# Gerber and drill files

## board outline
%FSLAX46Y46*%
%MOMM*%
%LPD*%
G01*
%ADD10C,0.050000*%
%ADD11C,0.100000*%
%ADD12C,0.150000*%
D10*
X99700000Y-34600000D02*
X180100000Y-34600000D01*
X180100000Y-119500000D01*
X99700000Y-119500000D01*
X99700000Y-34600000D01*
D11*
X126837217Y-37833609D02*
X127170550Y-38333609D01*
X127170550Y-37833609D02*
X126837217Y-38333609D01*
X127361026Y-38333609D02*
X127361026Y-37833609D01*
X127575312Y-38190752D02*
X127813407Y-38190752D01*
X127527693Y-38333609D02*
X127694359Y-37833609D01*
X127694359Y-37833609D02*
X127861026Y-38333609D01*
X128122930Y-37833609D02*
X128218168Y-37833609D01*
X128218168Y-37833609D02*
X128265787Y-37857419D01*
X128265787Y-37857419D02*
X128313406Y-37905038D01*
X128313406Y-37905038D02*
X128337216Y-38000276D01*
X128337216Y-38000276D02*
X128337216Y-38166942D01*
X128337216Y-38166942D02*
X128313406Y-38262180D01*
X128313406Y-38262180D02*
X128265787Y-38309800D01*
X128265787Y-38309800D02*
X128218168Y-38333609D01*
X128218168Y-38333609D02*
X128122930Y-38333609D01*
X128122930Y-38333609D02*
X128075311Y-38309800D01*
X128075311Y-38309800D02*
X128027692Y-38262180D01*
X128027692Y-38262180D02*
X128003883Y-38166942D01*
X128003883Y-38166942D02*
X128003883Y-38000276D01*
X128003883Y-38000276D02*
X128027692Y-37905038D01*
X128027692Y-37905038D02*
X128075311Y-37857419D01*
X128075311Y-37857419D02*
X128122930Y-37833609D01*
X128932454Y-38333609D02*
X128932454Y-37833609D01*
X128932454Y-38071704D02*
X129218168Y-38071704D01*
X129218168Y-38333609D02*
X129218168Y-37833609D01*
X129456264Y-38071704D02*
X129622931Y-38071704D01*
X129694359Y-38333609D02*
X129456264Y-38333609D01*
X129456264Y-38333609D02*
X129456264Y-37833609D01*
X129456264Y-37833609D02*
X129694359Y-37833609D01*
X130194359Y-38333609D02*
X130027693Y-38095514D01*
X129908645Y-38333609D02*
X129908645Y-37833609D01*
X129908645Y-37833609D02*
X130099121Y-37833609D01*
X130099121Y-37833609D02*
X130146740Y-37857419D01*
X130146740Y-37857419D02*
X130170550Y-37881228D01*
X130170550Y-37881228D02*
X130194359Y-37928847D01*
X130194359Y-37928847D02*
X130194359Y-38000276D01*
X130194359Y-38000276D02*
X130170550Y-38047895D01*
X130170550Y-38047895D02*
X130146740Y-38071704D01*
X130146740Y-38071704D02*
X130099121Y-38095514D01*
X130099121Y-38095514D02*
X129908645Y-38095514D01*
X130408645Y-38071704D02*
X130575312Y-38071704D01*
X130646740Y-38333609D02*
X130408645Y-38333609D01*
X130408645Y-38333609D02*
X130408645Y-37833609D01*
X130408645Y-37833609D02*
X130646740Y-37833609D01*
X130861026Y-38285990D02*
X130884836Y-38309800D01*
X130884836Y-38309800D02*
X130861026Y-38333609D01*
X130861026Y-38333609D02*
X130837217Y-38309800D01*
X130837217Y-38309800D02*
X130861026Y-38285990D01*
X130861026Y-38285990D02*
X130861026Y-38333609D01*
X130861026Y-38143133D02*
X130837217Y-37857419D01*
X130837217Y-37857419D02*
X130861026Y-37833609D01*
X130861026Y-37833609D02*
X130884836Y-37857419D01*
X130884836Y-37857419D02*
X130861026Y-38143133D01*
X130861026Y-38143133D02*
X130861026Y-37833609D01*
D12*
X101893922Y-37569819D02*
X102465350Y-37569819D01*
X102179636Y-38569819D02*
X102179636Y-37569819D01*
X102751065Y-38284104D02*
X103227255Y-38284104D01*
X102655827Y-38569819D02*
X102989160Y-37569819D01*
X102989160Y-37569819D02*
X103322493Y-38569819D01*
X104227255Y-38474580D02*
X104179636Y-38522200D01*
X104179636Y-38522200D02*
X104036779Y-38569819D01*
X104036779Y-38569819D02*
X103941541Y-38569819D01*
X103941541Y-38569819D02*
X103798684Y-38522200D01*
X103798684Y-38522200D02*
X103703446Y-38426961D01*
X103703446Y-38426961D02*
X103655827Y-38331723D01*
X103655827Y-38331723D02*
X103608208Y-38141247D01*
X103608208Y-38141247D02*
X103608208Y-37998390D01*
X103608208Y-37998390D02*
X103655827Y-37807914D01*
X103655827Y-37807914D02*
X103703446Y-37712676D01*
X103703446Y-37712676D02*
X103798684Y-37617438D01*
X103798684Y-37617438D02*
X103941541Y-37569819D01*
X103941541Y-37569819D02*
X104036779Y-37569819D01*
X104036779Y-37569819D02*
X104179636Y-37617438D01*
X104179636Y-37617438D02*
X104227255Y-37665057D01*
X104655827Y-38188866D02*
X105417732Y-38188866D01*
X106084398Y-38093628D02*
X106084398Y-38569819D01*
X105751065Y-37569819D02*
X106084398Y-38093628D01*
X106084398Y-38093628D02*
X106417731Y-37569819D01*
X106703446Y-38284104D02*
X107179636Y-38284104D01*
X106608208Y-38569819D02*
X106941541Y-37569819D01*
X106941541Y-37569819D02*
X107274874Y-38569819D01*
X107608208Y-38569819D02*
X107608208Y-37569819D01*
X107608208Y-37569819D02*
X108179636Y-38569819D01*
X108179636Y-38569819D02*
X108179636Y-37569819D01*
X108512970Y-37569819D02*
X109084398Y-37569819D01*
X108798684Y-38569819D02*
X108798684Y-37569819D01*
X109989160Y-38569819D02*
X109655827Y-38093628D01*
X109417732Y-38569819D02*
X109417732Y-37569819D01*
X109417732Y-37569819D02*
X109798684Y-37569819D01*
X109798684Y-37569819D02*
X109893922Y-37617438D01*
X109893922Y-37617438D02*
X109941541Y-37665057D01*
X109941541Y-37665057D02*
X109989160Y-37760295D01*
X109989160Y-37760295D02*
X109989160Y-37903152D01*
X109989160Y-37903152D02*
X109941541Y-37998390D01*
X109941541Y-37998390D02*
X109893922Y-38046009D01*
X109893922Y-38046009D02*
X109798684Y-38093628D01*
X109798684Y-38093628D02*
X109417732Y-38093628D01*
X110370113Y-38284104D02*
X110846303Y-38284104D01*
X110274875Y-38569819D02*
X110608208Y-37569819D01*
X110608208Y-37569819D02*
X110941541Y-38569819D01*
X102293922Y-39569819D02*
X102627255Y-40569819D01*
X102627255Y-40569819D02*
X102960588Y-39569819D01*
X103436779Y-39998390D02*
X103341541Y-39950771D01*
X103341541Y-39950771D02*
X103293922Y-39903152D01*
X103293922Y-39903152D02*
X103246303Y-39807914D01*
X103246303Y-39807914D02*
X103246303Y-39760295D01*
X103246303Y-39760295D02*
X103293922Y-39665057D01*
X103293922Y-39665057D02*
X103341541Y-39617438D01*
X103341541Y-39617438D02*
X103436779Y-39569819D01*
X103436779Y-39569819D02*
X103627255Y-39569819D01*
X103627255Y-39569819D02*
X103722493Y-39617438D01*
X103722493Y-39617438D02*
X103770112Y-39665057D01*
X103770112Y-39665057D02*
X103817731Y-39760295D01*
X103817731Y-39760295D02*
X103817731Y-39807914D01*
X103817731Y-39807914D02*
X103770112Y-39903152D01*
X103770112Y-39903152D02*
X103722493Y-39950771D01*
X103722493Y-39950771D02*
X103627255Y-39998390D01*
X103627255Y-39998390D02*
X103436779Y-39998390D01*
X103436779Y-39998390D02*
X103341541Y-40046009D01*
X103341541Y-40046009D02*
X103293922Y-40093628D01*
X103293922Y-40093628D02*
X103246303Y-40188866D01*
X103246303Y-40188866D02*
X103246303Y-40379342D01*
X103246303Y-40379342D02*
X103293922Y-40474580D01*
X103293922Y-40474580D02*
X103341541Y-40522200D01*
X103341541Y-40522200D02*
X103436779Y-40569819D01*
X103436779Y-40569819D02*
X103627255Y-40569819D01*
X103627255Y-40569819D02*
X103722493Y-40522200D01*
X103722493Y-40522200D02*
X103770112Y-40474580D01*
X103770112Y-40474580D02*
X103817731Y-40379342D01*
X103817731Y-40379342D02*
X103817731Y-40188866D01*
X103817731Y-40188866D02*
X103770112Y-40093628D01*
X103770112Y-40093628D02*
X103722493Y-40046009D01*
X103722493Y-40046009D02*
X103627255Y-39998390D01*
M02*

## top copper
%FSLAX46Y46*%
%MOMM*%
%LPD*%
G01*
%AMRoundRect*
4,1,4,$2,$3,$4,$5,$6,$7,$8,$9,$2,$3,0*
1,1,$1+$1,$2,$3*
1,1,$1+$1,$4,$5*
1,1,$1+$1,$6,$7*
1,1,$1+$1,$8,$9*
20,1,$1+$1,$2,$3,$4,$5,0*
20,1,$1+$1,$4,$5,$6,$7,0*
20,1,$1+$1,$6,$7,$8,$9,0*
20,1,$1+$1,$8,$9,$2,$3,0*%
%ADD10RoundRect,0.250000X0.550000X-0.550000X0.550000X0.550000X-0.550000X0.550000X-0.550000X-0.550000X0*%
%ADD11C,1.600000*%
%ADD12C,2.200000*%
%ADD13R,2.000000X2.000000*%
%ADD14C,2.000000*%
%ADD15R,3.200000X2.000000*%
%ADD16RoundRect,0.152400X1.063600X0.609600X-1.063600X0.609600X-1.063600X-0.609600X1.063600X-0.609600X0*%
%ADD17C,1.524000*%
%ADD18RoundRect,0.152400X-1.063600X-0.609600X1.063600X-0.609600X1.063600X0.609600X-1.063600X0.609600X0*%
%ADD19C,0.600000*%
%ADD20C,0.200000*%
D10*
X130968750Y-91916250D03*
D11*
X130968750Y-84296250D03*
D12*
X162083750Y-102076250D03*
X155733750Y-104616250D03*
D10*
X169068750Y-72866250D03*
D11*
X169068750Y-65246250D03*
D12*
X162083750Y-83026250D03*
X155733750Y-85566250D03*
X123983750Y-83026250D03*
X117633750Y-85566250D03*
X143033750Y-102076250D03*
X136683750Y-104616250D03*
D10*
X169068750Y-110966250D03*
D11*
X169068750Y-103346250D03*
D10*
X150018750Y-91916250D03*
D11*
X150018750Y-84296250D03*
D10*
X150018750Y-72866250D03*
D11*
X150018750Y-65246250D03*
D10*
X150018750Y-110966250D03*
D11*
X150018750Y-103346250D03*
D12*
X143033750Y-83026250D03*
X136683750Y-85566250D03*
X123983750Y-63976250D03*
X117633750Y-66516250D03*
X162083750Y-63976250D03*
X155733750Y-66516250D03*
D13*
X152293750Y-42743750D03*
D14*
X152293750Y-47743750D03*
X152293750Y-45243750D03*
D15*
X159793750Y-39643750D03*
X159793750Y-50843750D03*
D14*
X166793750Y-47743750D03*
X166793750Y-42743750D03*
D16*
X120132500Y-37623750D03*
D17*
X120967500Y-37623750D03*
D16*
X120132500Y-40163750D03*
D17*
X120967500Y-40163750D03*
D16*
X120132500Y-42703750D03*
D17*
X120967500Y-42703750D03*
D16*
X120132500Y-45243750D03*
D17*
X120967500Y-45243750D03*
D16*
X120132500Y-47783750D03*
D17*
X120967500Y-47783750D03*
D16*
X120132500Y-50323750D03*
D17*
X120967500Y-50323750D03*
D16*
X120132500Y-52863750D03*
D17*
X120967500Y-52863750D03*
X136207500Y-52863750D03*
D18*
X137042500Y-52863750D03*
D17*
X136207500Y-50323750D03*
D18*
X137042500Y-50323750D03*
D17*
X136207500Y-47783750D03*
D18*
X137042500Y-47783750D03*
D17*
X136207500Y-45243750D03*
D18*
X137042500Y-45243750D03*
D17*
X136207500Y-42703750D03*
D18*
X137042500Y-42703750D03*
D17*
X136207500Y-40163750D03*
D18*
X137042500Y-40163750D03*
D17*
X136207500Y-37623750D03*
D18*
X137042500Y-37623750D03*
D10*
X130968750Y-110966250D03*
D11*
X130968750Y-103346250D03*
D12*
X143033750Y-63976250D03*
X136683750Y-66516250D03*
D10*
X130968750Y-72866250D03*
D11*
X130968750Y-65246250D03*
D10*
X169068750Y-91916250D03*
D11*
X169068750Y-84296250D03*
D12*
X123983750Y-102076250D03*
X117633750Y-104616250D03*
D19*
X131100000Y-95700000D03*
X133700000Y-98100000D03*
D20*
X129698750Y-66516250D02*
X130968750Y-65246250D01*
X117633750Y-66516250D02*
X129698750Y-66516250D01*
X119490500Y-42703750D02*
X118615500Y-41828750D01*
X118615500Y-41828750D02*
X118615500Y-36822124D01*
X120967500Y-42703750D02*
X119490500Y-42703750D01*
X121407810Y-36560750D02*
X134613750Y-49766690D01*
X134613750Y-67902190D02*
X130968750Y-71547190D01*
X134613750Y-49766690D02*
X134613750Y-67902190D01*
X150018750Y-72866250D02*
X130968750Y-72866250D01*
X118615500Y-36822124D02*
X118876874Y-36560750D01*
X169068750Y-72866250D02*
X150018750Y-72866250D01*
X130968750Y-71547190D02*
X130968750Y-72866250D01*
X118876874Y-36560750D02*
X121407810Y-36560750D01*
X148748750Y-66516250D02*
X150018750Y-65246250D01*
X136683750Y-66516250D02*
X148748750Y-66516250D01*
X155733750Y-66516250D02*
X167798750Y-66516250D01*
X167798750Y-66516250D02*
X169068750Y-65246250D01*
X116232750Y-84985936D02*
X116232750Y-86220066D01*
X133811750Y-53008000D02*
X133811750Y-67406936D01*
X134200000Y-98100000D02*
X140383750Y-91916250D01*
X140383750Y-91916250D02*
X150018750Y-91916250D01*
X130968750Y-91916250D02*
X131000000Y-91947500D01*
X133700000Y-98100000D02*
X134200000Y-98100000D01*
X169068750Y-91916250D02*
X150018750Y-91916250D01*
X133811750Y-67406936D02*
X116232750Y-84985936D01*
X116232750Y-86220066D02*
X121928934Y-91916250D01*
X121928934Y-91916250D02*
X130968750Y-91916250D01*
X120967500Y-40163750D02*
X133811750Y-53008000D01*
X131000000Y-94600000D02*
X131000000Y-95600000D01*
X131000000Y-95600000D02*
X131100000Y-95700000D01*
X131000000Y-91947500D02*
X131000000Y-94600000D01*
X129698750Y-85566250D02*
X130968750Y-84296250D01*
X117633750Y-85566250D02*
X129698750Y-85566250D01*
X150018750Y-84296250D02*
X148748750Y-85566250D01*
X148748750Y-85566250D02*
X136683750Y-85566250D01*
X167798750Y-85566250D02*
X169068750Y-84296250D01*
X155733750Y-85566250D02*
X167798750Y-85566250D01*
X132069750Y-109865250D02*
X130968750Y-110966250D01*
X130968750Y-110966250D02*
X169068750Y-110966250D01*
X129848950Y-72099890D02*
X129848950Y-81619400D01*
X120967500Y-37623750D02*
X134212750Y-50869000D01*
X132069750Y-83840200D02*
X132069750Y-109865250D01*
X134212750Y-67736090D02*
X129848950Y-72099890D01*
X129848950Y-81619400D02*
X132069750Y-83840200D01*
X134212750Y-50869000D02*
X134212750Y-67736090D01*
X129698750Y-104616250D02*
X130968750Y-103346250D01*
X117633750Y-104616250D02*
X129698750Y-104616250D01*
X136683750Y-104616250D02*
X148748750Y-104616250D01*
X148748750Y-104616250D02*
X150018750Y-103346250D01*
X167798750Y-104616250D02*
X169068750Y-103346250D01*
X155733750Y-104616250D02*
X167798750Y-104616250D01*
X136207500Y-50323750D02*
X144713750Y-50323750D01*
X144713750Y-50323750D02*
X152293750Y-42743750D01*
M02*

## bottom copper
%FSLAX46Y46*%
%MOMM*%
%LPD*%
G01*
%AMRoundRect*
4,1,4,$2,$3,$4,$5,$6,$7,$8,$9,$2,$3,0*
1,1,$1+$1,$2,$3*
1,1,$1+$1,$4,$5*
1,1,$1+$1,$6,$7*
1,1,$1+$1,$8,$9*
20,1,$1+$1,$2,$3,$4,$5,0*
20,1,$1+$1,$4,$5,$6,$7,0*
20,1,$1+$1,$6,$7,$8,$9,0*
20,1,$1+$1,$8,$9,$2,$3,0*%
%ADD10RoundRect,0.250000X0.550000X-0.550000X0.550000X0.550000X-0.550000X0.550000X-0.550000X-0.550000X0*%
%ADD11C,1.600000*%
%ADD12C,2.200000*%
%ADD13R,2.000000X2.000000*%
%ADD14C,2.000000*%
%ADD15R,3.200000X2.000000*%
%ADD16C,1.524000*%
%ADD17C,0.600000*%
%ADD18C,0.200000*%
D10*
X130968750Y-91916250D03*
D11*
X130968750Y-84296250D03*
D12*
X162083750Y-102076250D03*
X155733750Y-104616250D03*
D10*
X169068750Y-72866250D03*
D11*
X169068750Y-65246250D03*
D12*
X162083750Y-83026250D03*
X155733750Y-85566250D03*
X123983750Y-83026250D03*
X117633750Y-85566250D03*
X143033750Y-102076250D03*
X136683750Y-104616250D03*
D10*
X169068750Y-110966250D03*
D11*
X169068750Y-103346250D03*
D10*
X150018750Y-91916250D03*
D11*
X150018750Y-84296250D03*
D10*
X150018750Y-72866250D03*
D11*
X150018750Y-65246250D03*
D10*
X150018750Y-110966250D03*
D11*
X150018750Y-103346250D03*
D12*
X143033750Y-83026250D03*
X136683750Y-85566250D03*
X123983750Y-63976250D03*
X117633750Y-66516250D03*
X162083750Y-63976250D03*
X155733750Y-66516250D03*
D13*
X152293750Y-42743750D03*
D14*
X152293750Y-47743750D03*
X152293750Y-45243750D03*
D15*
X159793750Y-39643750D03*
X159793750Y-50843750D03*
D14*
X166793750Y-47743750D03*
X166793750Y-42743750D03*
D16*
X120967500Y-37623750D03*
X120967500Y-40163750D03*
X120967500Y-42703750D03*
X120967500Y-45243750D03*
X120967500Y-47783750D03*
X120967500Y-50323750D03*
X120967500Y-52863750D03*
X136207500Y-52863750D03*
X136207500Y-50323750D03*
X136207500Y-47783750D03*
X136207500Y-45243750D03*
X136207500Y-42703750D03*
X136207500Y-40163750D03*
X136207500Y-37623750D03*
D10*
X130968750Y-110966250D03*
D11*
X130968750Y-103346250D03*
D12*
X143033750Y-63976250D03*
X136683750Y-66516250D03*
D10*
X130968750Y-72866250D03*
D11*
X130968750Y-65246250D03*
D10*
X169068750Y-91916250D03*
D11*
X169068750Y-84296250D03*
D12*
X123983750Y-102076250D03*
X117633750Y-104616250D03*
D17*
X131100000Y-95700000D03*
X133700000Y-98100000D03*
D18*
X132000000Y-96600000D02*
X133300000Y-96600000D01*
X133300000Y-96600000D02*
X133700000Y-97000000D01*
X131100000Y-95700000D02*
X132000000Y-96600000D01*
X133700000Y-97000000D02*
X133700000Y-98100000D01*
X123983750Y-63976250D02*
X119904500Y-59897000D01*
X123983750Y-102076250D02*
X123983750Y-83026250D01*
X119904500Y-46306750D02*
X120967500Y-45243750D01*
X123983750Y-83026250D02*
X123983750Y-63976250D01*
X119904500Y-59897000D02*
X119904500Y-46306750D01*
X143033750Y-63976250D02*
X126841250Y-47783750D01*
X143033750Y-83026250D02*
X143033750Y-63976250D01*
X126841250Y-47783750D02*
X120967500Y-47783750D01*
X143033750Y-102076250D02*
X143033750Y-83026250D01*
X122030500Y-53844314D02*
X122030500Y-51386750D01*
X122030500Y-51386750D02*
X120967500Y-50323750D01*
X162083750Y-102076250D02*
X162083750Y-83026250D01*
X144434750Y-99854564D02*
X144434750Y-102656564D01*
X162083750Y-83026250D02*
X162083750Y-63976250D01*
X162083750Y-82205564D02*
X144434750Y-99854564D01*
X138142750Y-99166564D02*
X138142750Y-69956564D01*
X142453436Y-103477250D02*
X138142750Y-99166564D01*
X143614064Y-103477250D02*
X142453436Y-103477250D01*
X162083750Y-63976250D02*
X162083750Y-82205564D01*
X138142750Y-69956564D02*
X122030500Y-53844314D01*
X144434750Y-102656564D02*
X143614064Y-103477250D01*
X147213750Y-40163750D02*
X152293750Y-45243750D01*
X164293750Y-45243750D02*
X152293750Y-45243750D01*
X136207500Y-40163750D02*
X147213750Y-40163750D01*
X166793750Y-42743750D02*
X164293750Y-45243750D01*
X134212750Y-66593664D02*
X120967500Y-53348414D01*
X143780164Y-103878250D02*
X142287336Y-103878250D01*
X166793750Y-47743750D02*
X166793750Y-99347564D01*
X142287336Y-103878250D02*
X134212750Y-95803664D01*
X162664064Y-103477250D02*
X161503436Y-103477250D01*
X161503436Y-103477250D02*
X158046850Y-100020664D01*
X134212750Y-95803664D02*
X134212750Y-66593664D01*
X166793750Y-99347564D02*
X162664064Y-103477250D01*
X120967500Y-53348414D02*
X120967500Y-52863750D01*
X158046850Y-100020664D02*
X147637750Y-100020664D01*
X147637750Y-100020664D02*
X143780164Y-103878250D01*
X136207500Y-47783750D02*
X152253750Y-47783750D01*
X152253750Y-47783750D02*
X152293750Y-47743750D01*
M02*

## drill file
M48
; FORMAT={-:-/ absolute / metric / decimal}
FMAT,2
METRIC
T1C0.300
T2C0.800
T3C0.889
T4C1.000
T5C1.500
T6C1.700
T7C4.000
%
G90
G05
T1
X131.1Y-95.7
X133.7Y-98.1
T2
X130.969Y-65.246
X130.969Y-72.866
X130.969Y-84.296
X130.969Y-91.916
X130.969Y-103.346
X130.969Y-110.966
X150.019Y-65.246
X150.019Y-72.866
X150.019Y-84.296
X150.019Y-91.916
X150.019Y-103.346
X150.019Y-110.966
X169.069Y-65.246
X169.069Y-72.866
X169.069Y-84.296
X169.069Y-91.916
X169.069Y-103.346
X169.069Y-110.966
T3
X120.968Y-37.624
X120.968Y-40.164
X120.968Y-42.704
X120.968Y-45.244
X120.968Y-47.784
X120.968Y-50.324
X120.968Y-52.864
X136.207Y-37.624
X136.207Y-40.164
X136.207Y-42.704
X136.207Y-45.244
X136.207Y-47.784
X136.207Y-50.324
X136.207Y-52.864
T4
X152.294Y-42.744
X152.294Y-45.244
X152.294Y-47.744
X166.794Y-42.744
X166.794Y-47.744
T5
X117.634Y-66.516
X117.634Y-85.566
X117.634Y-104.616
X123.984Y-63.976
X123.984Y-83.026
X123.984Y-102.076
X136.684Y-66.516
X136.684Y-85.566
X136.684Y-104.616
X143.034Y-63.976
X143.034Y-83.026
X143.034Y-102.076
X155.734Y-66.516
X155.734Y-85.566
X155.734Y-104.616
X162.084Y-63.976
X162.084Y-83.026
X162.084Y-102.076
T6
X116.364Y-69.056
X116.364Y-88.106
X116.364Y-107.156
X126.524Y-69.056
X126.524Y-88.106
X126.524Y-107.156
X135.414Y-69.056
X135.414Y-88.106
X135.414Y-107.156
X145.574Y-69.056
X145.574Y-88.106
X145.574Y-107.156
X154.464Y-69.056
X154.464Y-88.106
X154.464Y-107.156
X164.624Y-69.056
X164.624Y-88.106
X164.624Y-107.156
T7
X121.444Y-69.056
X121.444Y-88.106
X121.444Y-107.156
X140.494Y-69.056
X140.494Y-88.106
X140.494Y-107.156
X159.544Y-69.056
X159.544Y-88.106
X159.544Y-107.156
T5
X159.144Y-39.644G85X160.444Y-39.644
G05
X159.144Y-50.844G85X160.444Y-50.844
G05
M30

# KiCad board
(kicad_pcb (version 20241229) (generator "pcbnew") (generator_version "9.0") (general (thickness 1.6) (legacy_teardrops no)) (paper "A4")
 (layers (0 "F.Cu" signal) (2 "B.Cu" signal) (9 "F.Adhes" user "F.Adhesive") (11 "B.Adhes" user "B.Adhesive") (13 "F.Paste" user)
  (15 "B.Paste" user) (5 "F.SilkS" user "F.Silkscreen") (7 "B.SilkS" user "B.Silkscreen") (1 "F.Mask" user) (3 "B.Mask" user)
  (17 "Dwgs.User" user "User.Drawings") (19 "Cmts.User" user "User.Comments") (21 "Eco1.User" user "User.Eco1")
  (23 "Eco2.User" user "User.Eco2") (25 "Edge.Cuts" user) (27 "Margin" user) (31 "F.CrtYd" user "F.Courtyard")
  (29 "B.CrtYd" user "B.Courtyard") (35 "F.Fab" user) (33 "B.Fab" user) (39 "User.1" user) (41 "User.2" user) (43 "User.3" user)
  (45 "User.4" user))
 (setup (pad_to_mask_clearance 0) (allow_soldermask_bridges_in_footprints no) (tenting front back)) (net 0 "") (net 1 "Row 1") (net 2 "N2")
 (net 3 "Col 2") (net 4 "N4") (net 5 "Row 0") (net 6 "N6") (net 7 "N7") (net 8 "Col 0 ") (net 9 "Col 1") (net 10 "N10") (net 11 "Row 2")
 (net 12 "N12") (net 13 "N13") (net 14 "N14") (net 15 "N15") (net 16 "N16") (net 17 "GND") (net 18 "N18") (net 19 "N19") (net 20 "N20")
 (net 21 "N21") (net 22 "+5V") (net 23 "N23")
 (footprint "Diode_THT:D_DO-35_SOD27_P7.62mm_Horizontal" (layer "F.Cu") (at 130.96875 91.91625 90)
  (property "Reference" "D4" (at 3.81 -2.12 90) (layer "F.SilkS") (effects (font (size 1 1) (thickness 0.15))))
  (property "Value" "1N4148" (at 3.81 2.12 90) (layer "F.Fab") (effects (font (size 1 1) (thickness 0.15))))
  (pad "1" thru_hole roundrect (at 0 0 90) (size 1.6 1.6) (drill 0.8) (layers "*.Cu" "*.Mask") (remove_unused_layers no)
   (roundrect_rratio 0.15625) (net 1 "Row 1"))
  (pad "2" thru_hole circle (at 7.62 0 90) (size 1.6 1.6) (drill 0.8) (layers "*.Cu" "*.Mask") (remove_unused_layers no) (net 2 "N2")))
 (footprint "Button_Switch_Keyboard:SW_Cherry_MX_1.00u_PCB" (layer "F.Cu") (at 162.08375 102.07625)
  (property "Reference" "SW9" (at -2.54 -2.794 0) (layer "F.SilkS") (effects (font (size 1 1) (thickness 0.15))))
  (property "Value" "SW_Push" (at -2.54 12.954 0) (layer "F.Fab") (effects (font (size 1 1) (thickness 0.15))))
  (pad "" np_thru_hole circle (at -7.62 5.08) (size 1.7 1.7) (drill 1.7) (layers "*.Cu" "*.Mask"))
  (pad "" np_thru_hole circle (at -2.54 5.08) (size 4 4) (drill 4) (layers "*.Cu" "*.Mask"))
  (pad "" np_thru_hole circle (at 2.54 5.08) (size 1.7 1.7) (drill 1.7) (layers "*.Cu" "*.Mask"))
  (pad "1" thru_hole circle (at 0 0) (size 2.2 2.2) (drill 1.5) (layers "*.Cu" "*.Mask") (remove_unused_layers no) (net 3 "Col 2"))
  (pad "2" thru_hole circle (at -6.35 2.54) (size 2.2 2.2) (drill 1.5) (layers "*.Cu" "*.Mask") (remove_unused_layers no) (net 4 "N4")))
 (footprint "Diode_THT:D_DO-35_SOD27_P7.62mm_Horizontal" (layer "F.Cu") (at 169.06875 72.86625 90)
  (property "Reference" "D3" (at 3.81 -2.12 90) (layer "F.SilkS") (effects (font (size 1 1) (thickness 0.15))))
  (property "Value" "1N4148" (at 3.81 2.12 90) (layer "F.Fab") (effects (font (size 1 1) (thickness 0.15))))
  (pad "1" thru_hole roundrect (at 0 0 90) (size 1.6 1.6) (drill 0.8) (layers "*.Cu" "*.Mask") (remove_unused_layers no)
   (roundrect_rratio 0.15625) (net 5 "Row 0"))
  (pad "2" thru_hole circle (at 7.62 0 90) (size 1.6 1.6) (drill 0.8) (layers "*.Cu" "*.Mask") (remove_unused_layers no) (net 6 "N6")))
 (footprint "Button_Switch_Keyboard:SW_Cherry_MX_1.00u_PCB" (layer "F.Cu") (at 162.08375 83.02625)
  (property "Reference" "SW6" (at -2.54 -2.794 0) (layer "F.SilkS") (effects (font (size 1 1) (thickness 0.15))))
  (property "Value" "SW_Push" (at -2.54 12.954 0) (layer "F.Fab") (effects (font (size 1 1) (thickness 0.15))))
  (pad "" np_thru_hole circle (at -7.62 5.08) (size 1.7 1.7) (drill 1.7) (layers "*.Cu" "*.Mask"))
  (pad "" np_thru_hole circle (at -2.54 5.08) (size 4 4) (drill 4) (layers "*.Cu" "*.Mask"))
  (pad "" np_thru_hole circle (at 2.54 5.08) (size 1.7 1.7) (drill 1.7) (layers "*.Cu" "*.Mask"))
  (pad "1" thru_hole circle (at 0 0) (size 2.2 2.2) (drill 1.5) (layers "*.Cu" "*.Mask") (remove_unused_layers no) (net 3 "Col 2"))
  (pad "2" thru_hole circle (at -6.35 2.54) (size 2.2 2.2) (drill 1.5) (layers "*.Cu" "*.Mask") (remove_unused_layers no) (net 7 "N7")))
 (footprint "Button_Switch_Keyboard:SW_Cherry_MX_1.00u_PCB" (layer "F.Cu") (at 123.98375 83.02625)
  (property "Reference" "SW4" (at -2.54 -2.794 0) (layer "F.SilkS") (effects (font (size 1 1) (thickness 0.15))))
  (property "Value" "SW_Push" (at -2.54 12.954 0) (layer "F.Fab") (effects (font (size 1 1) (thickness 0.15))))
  (pad "" np_thru_hole circle (at -7.62 5.08) (size 1.7 1.7) (drill 1.7) (layers "*.Cu" "*.Mask"))
  (pad "" np_thru_hole circle (at -2.54 5.08) (size 4 4) (drill 4) (layers "*.Cu" "*.Mask"))
  (pad "" np_thru_hole circle (at 2.54 5.08) (size 1.7 1.7) (drill 1.7) (layers "*.Cu" "*.Mask"))
  (pad "1" thru_hole circle (at 0 0) (size 2.2 2.2) (drill 1.5) (layers "*.Cu" "*.Mask") (remove_unused_layers no) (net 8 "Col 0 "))
  (pad "2" thru_hole circle (at -6.35 2.54) (size 2.2 2.2) (drill 1.5) (layers "*.Cu" "*.Mask") (remove_unused_layers no) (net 2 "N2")))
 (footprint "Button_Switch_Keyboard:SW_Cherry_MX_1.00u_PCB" (layer "F.Cu") (at 143.03375 102.07625)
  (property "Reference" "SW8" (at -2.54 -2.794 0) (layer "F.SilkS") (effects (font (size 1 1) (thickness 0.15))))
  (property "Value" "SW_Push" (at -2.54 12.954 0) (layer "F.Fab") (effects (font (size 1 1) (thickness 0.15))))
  (pad "" np_thru_hole circle (at -7.62 5.08) (size 1.7 1.7) (drill 1.7) (layers "*.Cu" "*.Mask"))
  (pad "" np_thru_hole circle (at -2.54 5.08) (size 4 4) (drill 4) (layers "*.Cu" "*.Mask"))
  (pad "" np_thru_hole circle (at 2.54 5.08) (size 1.7 1.7) (drill 1.7) (layers "*.Cu" "*.Mask"))
  (pad "1" thru_hole circle (at 0 0) (size 2.2 2.2) (drill 1.5) (layers "*.Cu" "*.Mask") (remove_unused_layers no) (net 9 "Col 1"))
  (pad "2" thru_hole circle (at -6.35 2.54) (size 2.2 2.2) (drill 1.5) (layers "*.Cu" "*.Mask") (remove_unused_layers no) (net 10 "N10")))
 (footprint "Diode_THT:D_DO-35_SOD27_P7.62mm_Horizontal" (layer "F.Cu") (at 169.06875 110.96625 90)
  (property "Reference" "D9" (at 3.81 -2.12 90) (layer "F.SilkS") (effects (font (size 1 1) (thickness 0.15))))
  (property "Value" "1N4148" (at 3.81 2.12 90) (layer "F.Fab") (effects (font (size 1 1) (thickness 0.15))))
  (pad "1" thru_hole roundrect (at 0 0 90) (size 1.6 1.6) (drill 0.8) (layers "*.Cu" "*.Mask") (remove_unused_layers no)
   (roundrect_rratio 0.15625) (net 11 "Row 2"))
  (pad "2" thru_hole circle (at 7.62 0 90) (size 1.6 1.6) (drill 0.8) (layers "*.Cu" "*.Mask") (remove_unused_layers no) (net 4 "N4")))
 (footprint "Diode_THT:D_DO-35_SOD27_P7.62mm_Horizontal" (layer "F.Cu") (at 150.01875 91.91625 90)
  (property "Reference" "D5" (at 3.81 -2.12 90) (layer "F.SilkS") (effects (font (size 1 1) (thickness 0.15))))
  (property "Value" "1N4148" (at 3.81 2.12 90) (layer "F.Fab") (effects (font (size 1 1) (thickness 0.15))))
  (pad "1" thru_hole roundrect (at 0 0 90) (size 1.6 1.6) (drill 0.8) (layers "*.Cu" "*.Mask") (remove_unused_layers no)
   (roundrect_rratio 0.15625) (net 1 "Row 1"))
  (pad "2" thru_hole circle (at 7.62 0 90) (size 1.6 1.6) (drill 0.8) (layers "*.Cu" "*.Mask") (remove_unused_layers no) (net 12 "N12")))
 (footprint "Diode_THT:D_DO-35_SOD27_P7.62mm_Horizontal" (layer "F.Cu") (at 150.01875 72.86625 90)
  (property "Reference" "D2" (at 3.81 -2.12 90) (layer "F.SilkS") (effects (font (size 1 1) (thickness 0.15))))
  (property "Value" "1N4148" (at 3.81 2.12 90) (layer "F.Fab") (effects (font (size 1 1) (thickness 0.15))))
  (pad "1" thru_hole roundrect (at 0 0 90) (size 1.6 1.6) (drill 0.8) (layers "*.Cu" "*.Mask") (remove_unused_layers no)
   (roundrect_rratio 0.15625) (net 5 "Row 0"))
  (pad "2" thru_hole circle (at 7.62 0 90) (size 1.6 1.6) (drill 0.8) (layers "*.Cu" "*.Mask") (remove_unused_layers no) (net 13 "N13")))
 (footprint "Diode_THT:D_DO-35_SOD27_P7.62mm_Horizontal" (layer "F.Cu") (at 150.01875 110.96625 90)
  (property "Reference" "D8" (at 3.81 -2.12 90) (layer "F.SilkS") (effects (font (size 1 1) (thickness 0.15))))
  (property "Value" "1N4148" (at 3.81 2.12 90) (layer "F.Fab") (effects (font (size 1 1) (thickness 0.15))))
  (pad "1" thru_hole roundrect (at 0 0 90) (size 1.6 1.6) (drill 0.8) (layers "*.Cu" "*.Mask") (remove_unused_layers no)
   (roundrect_rratio 0.15625) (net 11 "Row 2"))
  (pad "2" thru_hole circle (at 7.62 0 90) (size 1.6 1.6) (drill 0.8) (layers "*.Cu" "*.Mask") (remove_unused_layers no) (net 10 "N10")))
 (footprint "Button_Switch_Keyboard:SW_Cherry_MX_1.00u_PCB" (layer "F.Cu") (at 143.03375 83.02625)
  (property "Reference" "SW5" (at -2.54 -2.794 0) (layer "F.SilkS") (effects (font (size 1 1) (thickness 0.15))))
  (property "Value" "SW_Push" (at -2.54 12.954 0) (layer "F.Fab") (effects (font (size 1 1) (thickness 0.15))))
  (pad "" np_thru_hole circle (at -7.62 5.08) (size 1.7 1.7) (drill 1.7) (layers "*.Cu" "*.Mask"))
  (pad "" np_thru_hole circle (at -2.54 5.08) (size 4 4) (drill 4) (layers "*.Cu" "*.Mask"))
  (pad "" np_thru_hole circle (at 2.54 5.08) (size 1.7 1.7) (drill 1.7) (layers "*.Cu" "*.Mask"))
  (pad "1" thru_hole circle (at 0 0) (size 2.2 2.2) (drill 1.5) (layers "*.Cu" "*.Mask") (remove_unused_layers no) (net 9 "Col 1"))
  (pad "2" thru_hole circle (at -6.35 2.54) (size 2.2 2.2) (drill 1.5) (layers "*.Cu" "*.Mask") (remove_unused_layers no) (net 12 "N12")))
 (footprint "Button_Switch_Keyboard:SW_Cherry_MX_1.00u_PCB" (layer "F.Cu") (at 123.98375 63.97625)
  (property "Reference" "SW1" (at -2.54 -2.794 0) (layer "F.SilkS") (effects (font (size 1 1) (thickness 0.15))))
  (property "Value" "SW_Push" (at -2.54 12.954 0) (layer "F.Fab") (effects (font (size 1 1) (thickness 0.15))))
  (pad "" np_thru_hole circle (at -7.62 5.08) (size 1.7 1.7) (drill 1.7) (layers "*.Cu" "*.Mask"))
  (pad "" np_thru_hole circle (at -2.54 5.08) (size 4 4) (drill 4) (layers "*.Cu" "*.Mask"))
  (pad "" np_thru_hole circle (at 2.54 5.08) (size 1.7 1.7) (drill 1.7) (layers "*.Cu" "*.Mask"))
  (pad "1" thru_hole circle (at 0 0) (size 2.2 2.2) (drill 1.5) (layers "*.Cu" "*.Mask") (remove_unused_layers no) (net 8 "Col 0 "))
  (pad "2" thru_hole circle (at -6.35 2.54) (size 2.2 2.2) (drill 1.5) (layers "*.Cu" "*.Mask") (remove_unused_layers no) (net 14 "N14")))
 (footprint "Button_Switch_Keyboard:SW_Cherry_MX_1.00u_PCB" (layer "F.Cu") (at 162.08375 63.97625)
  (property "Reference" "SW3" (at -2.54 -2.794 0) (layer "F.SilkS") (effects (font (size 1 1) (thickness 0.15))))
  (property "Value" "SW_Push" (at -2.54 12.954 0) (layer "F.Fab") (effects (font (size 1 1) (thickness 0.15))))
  (pad "" np_thru_hole circle (at -7.62 5.08) (size 1.7 1.7) (drill 1.7) (layers "*.Cu" "*.Mask"))
  (pad "" np_thru_hole circle (at -2.54 5.08) (size 4 4) (drill 4) (layers "*.Cu" "*.Mask"))
  (pad "" np_thru_hole circle (at 2.54 5.08) (size 1.7 1.7) (drill 1.7) (layers "*.Cu" "*.Mask"))
  (pad "1" thru_hole circle (at 0 0) (size 2.2 2.2) (drill 1.5) (layers "*.Cu" "*.Mask") (remove_unused_layers no) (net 3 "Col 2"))
  (pad "2" thru_hole circle (at -6.35 2.54) (size 2.2 2.2) (drill 1.5) (layers "*.Cu" "*.Mask") (remove_unused_layers no) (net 6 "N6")))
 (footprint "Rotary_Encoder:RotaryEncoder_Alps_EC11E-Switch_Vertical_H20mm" (layer "F.Cu") (at 152.29375 42.74375)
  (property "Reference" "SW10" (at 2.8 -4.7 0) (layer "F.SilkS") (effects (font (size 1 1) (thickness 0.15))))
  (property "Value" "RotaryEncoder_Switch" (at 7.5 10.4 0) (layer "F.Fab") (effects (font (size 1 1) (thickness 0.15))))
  (pad "A" thru_hole rect (at 0 0) (size 2 2) (drill 1) (layers "*.Cu" "*.Mask") (remove_unused_layers no) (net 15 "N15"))
  (pad "B" thru_hole circle (at 0 5) (size 2 2) (drill 1) (layers "*.Cu" "*.Mask") (remove_unused_layers no) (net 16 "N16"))
  (pad "C" thru_hole circle (at 0 2.5) (size 2 2) (drill 1) (layers "*.Cu" "*.Mask") (remove_unused_layers no) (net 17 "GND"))
  (pad "MP" thru_hole rect (at 7.5 -3.1) (size 3.2 2) (drill oval 2.8 1.5) (layers "*.Cu" "*.Mask") (remove_unused_layers no))
  (pad "MP" thru_hole rect (at 7.5 8.1) (size 3.2 2) (drill oval 2.8 1.5) (layers "*.Cu" "*.Mask") (remove_unused_layers no))
  (pad "S1" thru_hole circle (at 14.5 5) (size 2 2) (drill 1) (layers "*.Cu" "*.Mask") (remove_unused_layers no) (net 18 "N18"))
  (pad "S2" thru_hole circle (at 14.5 0) (size 2 2) (drill 1) (layers "*.Cu" "*.Mask") (remove_unused_layers no) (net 17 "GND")))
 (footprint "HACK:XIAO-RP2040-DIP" (layer "F.Cu") (at 128.5875 45.24375)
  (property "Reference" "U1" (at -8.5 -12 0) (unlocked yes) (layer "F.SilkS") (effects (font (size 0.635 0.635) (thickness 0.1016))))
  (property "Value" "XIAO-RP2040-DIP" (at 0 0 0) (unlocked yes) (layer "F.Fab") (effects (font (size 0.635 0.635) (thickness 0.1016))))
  (pad "1" smd roundrect (at -8.455 -7.62 180) (size 2.432 1.524) (layers "F.Cu" "F.Mask") (roundrect_rratio 0.1) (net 11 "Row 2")
   (thermal_bridge_angle 45))
  (pad "1" thru_hole circle (at -7.62 -7.62 180) (size 1.524 1.524) (drill 0.889) (layers "*.Cu" "*.Mask") (remove_unused_layers no)
   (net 11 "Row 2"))
  (pad "2" smd roundrect (at -8.455 -5.08 180) (size 2.432 1.524) (layers "F.Cu" "F.Mask") (roundrect_rratio 0.1) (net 1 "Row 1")
   (thermal_bridge_angle 45))
  (pad "2" thru_hole circle (at -7.62 -5.08 180) (size 1.524 1.524) (drill 0.889) (layers "*.Cu" "*.Mask") (remove_unused_layers no)
   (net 1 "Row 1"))
  (pad "3" smd roundrect (at -8.455 -2.54 180) (size 2.432 1.524) (layers "F.Cu" "F.Mask") (roundrect_rratio 0.1) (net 5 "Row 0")
   (thermal_bridge_angle 45))
  (pad "3" thru_hole circle (at -7.62 -2.54 180) (size 1.524 1.524) (drill 0.889) (layers "*.Cu" "*.Mask") (remove_unused_layers no)
   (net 5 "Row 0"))
  (pad "4" smd roundrect (at -8.455 0 180) (size 2.432 1.524) (layers "F.Cu" "F.Mask") (roundrect_rratio 0.1) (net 8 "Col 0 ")
   (thermal_bridge_angle 45))
  (pad "4" thru_hole circle (at -7.62 0 180) (size 1.524 1.524) (drill 0.889) (layers "*.Cu" "*.Mask") (remove_unused_layers no)
   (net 8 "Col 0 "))
  (pad "5" smd roundrect (at -8.455 2.54 180) (size 2.432 1.524) (layers "F.Cu" "F.Mask") (roundrect_rratio 0.1) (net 9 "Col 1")
   (thermal_bridge_angle 45))
  (pad "5" thru_hole circle (at -7.62 2.54 180) (size 1.524 1.524) (drill 0.889) (layers "*.Cu" "*.Mask") (remove_unused_layers no)
   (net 9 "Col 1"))
  (pad "6" smd roundrect (at -8.455 5.08 180) (size 2.432 1.524) (layers "F.Cu" "F.Mask") (roundrect_rratio 0.1) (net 3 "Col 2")
   (thermal_bridge_angle 45))
  (pad "6" thru_hole circle (at -7.62 5.08 180) (size 1.524 1.524) (drill 0.889) (layers "*.Cu" "*.Mask") (remove_unused_layers no)
   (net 3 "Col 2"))
  (pad "7" smd roundrect (at -8.455 7.62 180) (size 2.432 1.524) (layers "F.Cu" "F.Mask") (roundrect_rratio 0.1) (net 18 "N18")
   (thermal_bridge_angle 45))
  (pad "7" thru_hole circle (at -7.62 7.62 180) (size 1.524 1.524) (drill 0.889) (layers "*.Cu" "*.Mask") (remove_unused_layers no)
   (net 18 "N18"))
  (pad "8" thru_hole circle (at 7.62 7.62) (size 1.524 1.524) (drill 0.889) (layers "*.Cu" "*.Mask") (remove_unused_layers no)
   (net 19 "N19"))
  (pad "8" smd roundrect (at 8.455 7.62) (size 2.432 1.524) (layers "F.Cu" "F.Mask") (roundrect_rratio 0.1) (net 19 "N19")
   (thermal_bridge_angle 45))
  (pad "9" thru_hole circle (at 7.62 5.08) (size 1.524 1.524) (drill 0.889) (layers "*.Cu" "*.Mask") (remove_unused_layers no)
   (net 15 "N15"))
  (pad "9" smd roundrect (at 8.455 5.08) (size 2.432 1.524) (layers "F.Cu" "F.Mask") (roundrect_rratio 0.1) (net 15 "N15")
   (thermal_bridge_angle 45))
  (pad "10" thru_hole circle (at 7.62 2.54) (size 1.524 1.524) (drill 0.889) (layers "*.Cu" "*.Mask") (remove_unused_layers no)
   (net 16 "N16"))
  (pad "10" smd roundrect (at 8.455 2.54) (size 2.432 1.524) (layers "F.Cu" "F.Mask") (roundrect_rratio 0.1) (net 16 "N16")
   (thermal_bridge_angle 45))
  (pad "11" thru_hole circle (at 7.62 0) (size 1.524 1.524) (drill 0.889) (layers "*.Cu" "*.Mask") (remove_unused_layers no) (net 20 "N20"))
  (pad "11" smd roundrect (at 8.455 0) (size 2.432 1.524) (layers "F.Cu" "F.Mask") (roundrect_rratio 0.1) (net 20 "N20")
   (thermal_bridge_angle 45))
  (pad "12" thru_hole circle (at 7.62 -2.54) (size 1.524 1.524) (drill 0.889) (layers "*.Cu" "*.Mask") (remove_unused_layers no)
   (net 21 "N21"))
  (pad "12" smd roundrect (at 8.455 -2.54) (size 2.432 1.524) (layers "F.Cu" "F.Mask") (roundrect_rratio 0.1) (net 21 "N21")
   (thermal_bridge_angle 45))
  (pad "13" thru_hole circle (at 7.62 -5.08) (size 1.524 1.524) (drill 0.889) (layers "*.Cu" "*.Mask") (remove_unused_layers no)
   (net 17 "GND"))
  (pad "13" smd roundrect (at 8.455 -5.08) (size 2.432 1.524) (layers "F.Cu" "F.Mask") (roundrect_rratio 0.1) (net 17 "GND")
   (thermal_bridge_angle 45))
  (pad "14" thru_hole circle (at 7.62 -7.62) (size 1.524 1.524) (drill 0.889) (layers "*.Cu" "*.Mask") (remove_unused_layers no)
   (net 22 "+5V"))
  (pad "14" smd roundrect (at 8.455 -7.62) (size 2.432 1.524) (layers "F.Cu" "F.Mask") (roundrect_rratio 0.1) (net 22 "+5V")
   (thermal_bridge_angle 45)))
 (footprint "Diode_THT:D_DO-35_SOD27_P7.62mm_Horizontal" (layer "F.Cu") (at 130.96875 110.96625 90)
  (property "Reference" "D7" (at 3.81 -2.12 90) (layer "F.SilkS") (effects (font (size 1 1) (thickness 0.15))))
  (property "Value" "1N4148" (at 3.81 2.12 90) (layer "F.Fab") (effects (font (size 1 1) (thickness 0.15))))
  (pad "1" thru_hole roundrect (at 0 0 90) (size 1.6 1.6) (drill 0.8) (layers "*.Cu" "*.Mask") (remove_unused_layers no)
   (roundrect_rratio 0.15625) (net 11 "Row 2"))
  (pad "2" thru_hole circle (at 7.62 0 90) (size 1.6 1.6) (drill 0.8) (layers "*.Cu" "*.Mask") (remove_unused_layers no) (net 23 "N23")))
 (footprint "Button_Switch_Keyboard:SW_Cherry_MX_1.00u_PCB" (layer "F.Cu") (at 143.03375 63.97625)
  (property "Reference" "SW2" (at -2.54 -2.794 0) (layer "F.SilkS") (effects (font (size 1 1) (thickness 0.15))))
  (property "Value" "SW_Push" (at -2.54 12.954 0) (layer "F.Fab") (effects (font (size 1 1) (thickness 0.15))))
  (pad "" np_thru_hole circle (at -7.62 5.08) (size 1.7 1.7) (drill 1.7) (layers "*.Cu" "*.Mask"))
  (pad "" np_thru_hole circle (at -2.54 5.08) (size 4 4) (drill 4) (layers "*.Cu" "*.Mask"))
  (pad "" np_thru_hole circle (at 2.54 5.08) (size 1.7 1.7) (drill 1.7) (layers "*.Cu" "*.Mask"))
  (pad "1" thru_hole circle (at 0 0) (size 2.2 2.2) (drill 1.5) (layers "*.Cu" "*.Mask") (remove_unused_layers no) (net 9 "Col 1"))
  (pad "2" thru_hole circle (at -6.35 2.54) (size 2.2 2.2) (drill 1.5) (layers "*.Cu" "*.Mask") (remove_unused_layers no) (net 13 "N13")))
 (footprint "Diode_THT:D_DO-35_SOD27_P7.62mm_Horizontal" (layer "F.Cu") (at 130.96875 72.86625 90)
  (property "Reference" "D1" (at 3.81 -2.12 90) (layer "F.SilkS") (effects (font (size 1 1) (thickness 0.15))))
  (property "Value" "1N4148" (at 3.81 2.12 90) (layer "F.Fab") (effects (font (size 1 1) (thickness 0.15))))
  (pad "1" thru_hole roundrect (at 0 0 90) (size 1.6 1.6) (drill 0.8) (layers "*.Cu" "*.Mask") (remove_unused_layers no)
   (roundrect_rratio 0.15625) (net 5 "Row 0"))
  (pad "2" thru_hole circle (at 7.62 0 90) (size 1.6 1.6) (drill 0.8) (layers "*.Cu" "*.Mask") (remove_unused_layers no) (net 14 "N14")))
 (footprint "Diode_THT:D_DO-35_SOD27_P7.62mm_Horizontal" (layer "F.Cu") (at 169.06875 91.91625 90)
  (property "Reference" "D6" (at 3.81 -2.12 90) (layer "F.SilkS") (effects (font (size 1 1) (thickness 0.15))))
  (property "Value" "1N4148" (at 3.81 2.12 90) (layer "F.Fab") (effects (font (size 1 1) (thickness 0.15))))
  (pad "1" thru_hole roundrect (at 0 0 90) (size 1.6 1.6) (drill 0.8) (layers "*.Cu" "*.Mask") (remove_unused_layers no)
   (roundrect_rratio 0.15625) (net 1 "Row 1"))
  (pad "2" thru_hole circle (at 7.62 0 90) (size 1.6 1.6) (drill 0.8) (layers "*.Cu" "*.Mask") (remove_unused_layers no) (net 7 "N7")))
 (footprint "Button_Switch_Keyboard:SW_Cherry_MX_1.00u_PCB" (layer "F.Cu") (at 123.98375 102.07625)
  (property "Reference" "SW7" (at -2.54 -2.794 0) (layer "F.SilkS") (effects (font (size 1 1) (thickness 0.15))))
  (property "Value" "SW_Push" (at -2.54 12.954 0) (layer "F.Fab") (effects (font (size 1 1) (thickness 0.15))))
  (pad "" np_thru_hole circle (at -7.62 5.08) (size 1.7 1.7) (drill 1.7) (layers "*.Cu" "*.Mask"))
  (pad "" np_thru_hole circle (at -2.54 5.08) (size 4 4) (drill 4) (layers "*.Cu" "*.Mask"))
  (pad "" np_thru_hole circle (at 2.54 5.08) (size 1.7 1.7) (drill 1.7) (layers "*.Cu" "*.Mask"))
  (pad "1" thru_hole circle (at 0 0) (size 2.2 2.2) (drill 1.5) (layers "*.Cu" "*.Mask") (remove_unused_layers no) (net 8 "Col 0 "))
  (pad "2" thru_hole circle (at -6.35 2.54) (size 2.2 2.2) (drill 1.5) (layers "*.Cu" "*.Mask") (remove_unused_layers no) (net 23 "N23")))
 (gr_rect (start 99.7 34.6) (end 180.1 119.5) (stroke (width 0.05) (type default)) (fill no) (layer "Edge.Cuts"))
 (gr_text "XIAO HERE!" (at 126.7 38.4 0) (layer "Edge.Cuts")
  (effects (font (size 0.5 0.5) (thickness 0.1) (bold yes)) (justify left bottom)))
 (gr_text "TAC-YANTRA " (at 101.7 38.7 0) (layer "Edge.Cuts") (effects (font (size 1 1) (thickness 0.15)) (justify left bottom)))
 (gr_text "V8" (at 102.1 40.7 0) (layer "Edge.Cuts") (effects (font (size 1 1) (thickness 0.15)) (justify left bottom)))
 (segment (start 129.69875 66.51625) (end 130.96875 65.24625) (width 0.2) (layer "F.Cu") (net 14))
 (segment (start 117.63375 66.51625) (end 129.69875 66.51625) (width 0.2) (layer "F.Cu") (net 14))
 (segment (start 119.4905 42.70375) (end 118.6155 41.82875) (width 0.2) (layer "F.Cu") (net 5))
 (segment (start 118.6155 41.82875) (end 118.6155 36.822124) (width 0.2) (layer "F.Cu") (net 5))
 (segment (start 120.9675 42.70375) (end 119.4905 42.70375) (width 0.2) (layer "F.Cu") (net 5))
 (segment (start 121.40781 36.56075) (end 134.61375 49.76669) (width 0.2) (layer "F.Cu") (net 5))
 (segment (start 134.61375 67.90219) (end 130.96875 71.54719) (width 0.2) (layer "F.Cu") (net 5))
 (segment (start 134.61375 49.76669) (end 134.61375 67.90219) (width 0.2) (layer "F.Cu") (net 5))
 (segment (start 150.01875 72.86625) (end 130.96875 72.86625) (width 0.2) (layer "F.Cu") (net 5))
 (segment (start 118.6155 36.822124) (end 118.876874 36.56075) (width 0.2) (layer "F.Cu") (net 5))
 (segment (start 169.06875 72.86625) (end 150.01875 72.86625) (width 0.2) (layer "F.Cu") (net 5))
 (segment (start 130.96875 71.54719) (end 130.96875 72.86625) (width 0.2) (layer "F.Cu") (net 5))
 (segment (start 118.876874 36.56075) (end 121.40781 36.56075) (width 0.2) (layer "F.Cu") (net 5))
 (segment (start 148.74875 66.51625) (end 150.01875 65.24625) (width 0.2) (layer "F.Cu") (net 13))
 (segment (start 136.68375 66.51625) (end 148.74875 66.51625) (width 0.2) (layer "F.Cu") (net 13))
 (segment (start 155.73375 66.51625) (end 167.79875 66.51625) (width 0.2) (layer "F.Cu") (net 6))
 (segment (start 167.79875 66.51625) (end 169.06875 65.24625) (width 0.2) (layer "F.Cu") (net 6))
 (segment (start 116.23275 84.985936) (end 116.23275 86.220066) (width 0.2) (layer "F.Cu") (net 1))
 (segment (start 133.81175 53.008) (end 133.81175 67.406936) (width 0.2) (layer "F.Cu") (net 1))
 (segment (start 134.2 98.1) (end 140.38375 91.91625) (width 0.2) (layer "F.Cu") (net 1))
 (segment (start 140.38375 91.91625) (end 150.01875 91.91625) (width 0.2) (layer "F.Cu") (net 1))
 (segment (start 130.96875 91.91625) (end 131 91.9475) (width 0.2) (layer "F.Cu") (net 1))
 (segment (start 133.7 98.1) (end 134.2 98.1) (width 0.2) (layer "F.Cu") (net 1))
 (segment (start 169.06875 91.91625) (end 150.01875 91.91625) (width 0.2) (layer "F.Cu") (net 1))
 (segment (start 133.81175 67.406936) (end 116.23275 84.985936) (width 0.2) (layer "F.Cu") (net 1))
 (segment (start 116.23275 86.220066) (end 121.928934 91.91625) (width 0.2) (layer "F.Cu") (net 1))
 (segment (start 121.928934 91.91625) (end 130.96875 91.91625) (width 0.2) (layer "F.Cu") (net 1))
 (segment (start 120.9675 40.16375) (end 133.81175 53.008) (width 0.2) (layer "F.Cu") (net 1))
 (segment (start 131 94.6) (end 131 95.6) (width 0.2) (layer "F.Cu") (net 1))
 (segment (start 131 95.6) (end 131.1 95.7) (width 0.2) (layer "F.Cu") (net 1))
 (segment (start 131 91.9475) (end 131 94.6) (width 0.2) (layer "F.Cu") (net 1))
 (via (at 131.1 95.7) (size 0.6) (drill 0.3) (layers "F.Cu" "B.Cu") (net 1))
 (via (at 133.7 98.1) (size 0.6) (drill 0.3) (layers "F.Cu" "B.Cu") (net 1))
 (segment (start 132 96.6) (end 133.3 96.6) (width 0.2) (layer "B.Cu") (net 1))
 (segment (start 133.3 96.6) (end 133.7 97) (width 0.2) (layer "B.Cu") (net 1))
 (segment (start 131.1 95.7) (end 132 96.6) (width 0.2) (layer "B.Cu") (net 1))
 (segment (start 133.7 97) (end 133.7 98.1) (width 0.2) (layer "B.Cu") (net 1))
 (segment (start 129.69875 85.56625) (end 130.96875 84.29625) (width 0.2) (layer "F.Cu") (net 2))
 (segment (start 117.63375 85.56625) (end 129.69875 85.56625) (width 0.2) (layer "F.Cu") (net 2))
 (segment (start 150.01875 84.29625) (end 148.74875 85.56625) (width 0.2) (layer "F.Cu") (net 12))
 (segment (start 148.74875 85.56625) (end 136.68375 85.56625) (width 0.2) (layer "F.Cu") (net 12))
 (segment (start 167.79875 85.56625) (end 169.06875 84.29625) (width 0.2) (layer "F.Cu") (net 7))
 (segment (start 155.73375 85.56625) (end 167.79875 85.56625) (width 0.2) (layer "F.Cu") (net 7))
 (segment (start 132.06975 109.86525) (end 130.96875 110.96625) (width 0.2) (layer "F.Cu") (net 11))
 (segment (start 130.96875 110.96625) (end 169.06875 110.96625) (width 0.2) (layer "F.Cu") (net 11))
 (segment (start 129.84895 72.09989) (end 129.84895 81.6194) (width 0.2) (layer "F.Cu") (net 11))
 (segment (start 120.9675 37.62375) (end 134.21275 50.869) (width 0.2) (layer "F.Cu") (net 11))
 (segment (start 132.06975 83.8402) (end 132.06975 109.86525) (width 0.2) (layer "F.Cu") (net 11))
 (segment (start 134.21275 67.73609) (end 129.84895 72.09989) (width 0.2) (layer "F.Cu") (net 11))
 (segment (start 129.84895 81.6194) (end 132.06975 83.8402) (width 0.2) (layer "F.Cu") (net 11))
 (segment (start 134.21275 50.869) (end 134.21275 67.73609) (width 0.2) (layer "F.Cu") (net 11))
 (segment (start 129.69875 104.61625) (end 130.96875 103.34625) (width 0.2) (layer "F.Cu") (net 23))
 (segment (start 117.63375 104.61625) (end 129.69875 104.61625) (width 0.2) (layer "F.Cu") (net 23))
 (segment (start 136.68375 104.61625) (end 148.74875 104.61625) (width 0.2) (layer "F.Cu") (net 10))
 (segment (start 148.74875 104.61625) (end 150.01875 103.34625) (width 0.2) (layer "F.Cu") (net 10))
 (segment (start 167.79875 104.61625) (end 169.06875 103.34625) (width 0.2) (layer "F.Cu") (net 4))
 (segment (start 155.73375 104.61625) (end 167.79875 104.61625) (width 0.2) (layer "F.Cu") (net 4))
 (segment (start 123.98375 63.97625) (end 119.9045 59.897) (width 0.2) (layer "B.Cu") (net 8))
 (segment (start 123.98375 102.07625) (end 123.98375 83.02625) (width 0.2) (layer "B.Cu") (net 8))
 (segment (start 119.9045 46.30675) (end 120.9675 45.24375) (width 0.2) (layer "B.Cu") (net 8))
 (segment (start 123.98375 83.02625) (end 123.98375 63.97625) (width 0.2) (layer "B.Cu") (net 8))
 (segment (start 119.9045 59.897) (end 119.9045 46.30675) (width 0.2) (layer "B.Cu") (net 8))
 (segment (start 143.03375 63.97625) (end 126.84125 47.78375) (width 0.2) (layer "B.Cu") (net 9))
 (segment (start 143.03375 83.02625) (end 143.03375 63.97625) (width 0.2) (layer "B.Cu") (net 9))
 (segment (start 126.84125 47.78375) (end 120.9675 47.78375) (width 0.2) (layer "B.Cu") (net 9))
 (segment (start 143.03375 102.07625) (end 143.03375 83.02625) (width 0.2) (layer "B.Cu") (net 9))
 (segment (start 122.0305 53.844314) (end 122.0305 51.38675) (width 0.2) (layer "B.Cu") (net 3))
 (segment (start 122.0305 51.38675) (end 120.9675 50.32375) (width 0.2) (layer "B.Cu") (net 3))
 (segment (start 162.08375 102.07625) (end 162.08375 83.02625) (width 0.2) (layer "B.Cu") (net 3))
 (segment (start 144.43475 99.854564) (end 144.43475 102.656564) (width 0.2) (layer "B.Cu") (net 3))
 (segment (start 162.08375 83.02625) (end 162.08375 63.97625) (width 0.2) (layer "B.Cu") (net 3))
 (segment (start 162.08375 82.205564) (end 144.43475 99.854564) (width 0.2) (layer "B.Cu") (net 3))
 (segment (start 138.14275 99.166564) (end 138.14275 69.956564) (width 0.2) (layer "B.Cu") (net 3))
 (segment (start 142.453436 103.47725) (end 138.14275 99.166564) (width 0.2) (layer "B.Cu") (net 3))
 (segment (start 143.614064 103.47725) (end 142.453436 103.47725) (width 0.2) (layer "B.Cu") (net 3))
 (segment (start 162.08375 63.97625) (end 162.08375 82.205564) (width 0.2) (layer "B.Cu") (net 3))
 (segment (start 138.14275 69.956564) (end 122.0305 53.844314) (width 0.2) (layer "B.Cu") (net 3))
 (segment (start 144.43475 102.656564) (end 143.614064 103.47725) (width 0.2) (layer "B.Cu") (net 3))
 (segment (start 147.21375 40.16375) (end 152.29375 45.24375) (width 0.2) (layer "B.Cu") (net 17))
 (segment (start 164.29375 45.24375) (end 152.29375 45.24375) (width 0.2) (layer "B.Cu") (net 17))
 (segment (start 136.2075 40.16375) (end 147.21375 40.16375) (width 0.2) (layer "B.Cu") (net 17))
 (segment (start 166.79375 42.74375) (end 164.29375 45.24375) (width 0.2) (layer "B.Cu") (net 17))
 (segment (start 136.2075 50.32375) (end 144.71375 50.32375) (width 0.2) (layer "F.Cu") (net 15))
 (segment (start 144.71375 50.32375) (end 152.29375 42.74375) (width 0.2) (layer "F.Cu") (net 15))
 (segment (start 134.21275 66.593664) (end 120.9675 53.348414) (width 0.2) (layer "B.Cu") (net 18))
 (segment (start 143.780164 103.87825) (end 142.287336 103.87825) (width 0.2) (layer "B.Cu") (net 18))
 (segment (start 166.79375 47.74375) (end 166.79375 99.347564) (width 0.2) (layer "B.Cu") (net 18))
 (segment (start 142.287336 103.87825) (end 134.21275 95.803664) (width 0.2) (layer "B.Cu") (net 18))
 (segment (start 162.664064 103.47725) (end 161.503436 103.47725) (width 0.2) (layer "B.Cu") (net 18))
 (segment (start 161.503436 103.47725) (end 158.04685 100.020664) (width 0.2) (layer "B.Cu") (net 18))
 (segment (start 134.21275 95.803664) (end 134.21275 66.593664) (width 0.2) (layer "B.Cu") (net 18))
 (segment (start 166.79375 99.347564) (end 162.664064 103.47725) (width 0.2) (layer "B.Cu") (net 18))
 (segment (start 120.9675 53.348414) (end 120.9675 52.86375) (width 0.2) (layer "B.Cu") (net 18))
 (segment (start 158.04685 100.020664) (end 147.63775 100.020664) (width 0.2) (layer "B.Cu") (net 18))
 (segment (start 147.63775 100.020664) (end 143.780164 103.87825) (width 0.2) (layer "B.Cu") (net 18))
 (segment (start 136.2075 47.78375) (end 152.25375 47.78375) (width 0.2) (layer "B.Cu") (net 16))
 (segment (start 152.25375 47.78375) (end 152.29375 47.74375) (width 0.2) (layer "B.Cu") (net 16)))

